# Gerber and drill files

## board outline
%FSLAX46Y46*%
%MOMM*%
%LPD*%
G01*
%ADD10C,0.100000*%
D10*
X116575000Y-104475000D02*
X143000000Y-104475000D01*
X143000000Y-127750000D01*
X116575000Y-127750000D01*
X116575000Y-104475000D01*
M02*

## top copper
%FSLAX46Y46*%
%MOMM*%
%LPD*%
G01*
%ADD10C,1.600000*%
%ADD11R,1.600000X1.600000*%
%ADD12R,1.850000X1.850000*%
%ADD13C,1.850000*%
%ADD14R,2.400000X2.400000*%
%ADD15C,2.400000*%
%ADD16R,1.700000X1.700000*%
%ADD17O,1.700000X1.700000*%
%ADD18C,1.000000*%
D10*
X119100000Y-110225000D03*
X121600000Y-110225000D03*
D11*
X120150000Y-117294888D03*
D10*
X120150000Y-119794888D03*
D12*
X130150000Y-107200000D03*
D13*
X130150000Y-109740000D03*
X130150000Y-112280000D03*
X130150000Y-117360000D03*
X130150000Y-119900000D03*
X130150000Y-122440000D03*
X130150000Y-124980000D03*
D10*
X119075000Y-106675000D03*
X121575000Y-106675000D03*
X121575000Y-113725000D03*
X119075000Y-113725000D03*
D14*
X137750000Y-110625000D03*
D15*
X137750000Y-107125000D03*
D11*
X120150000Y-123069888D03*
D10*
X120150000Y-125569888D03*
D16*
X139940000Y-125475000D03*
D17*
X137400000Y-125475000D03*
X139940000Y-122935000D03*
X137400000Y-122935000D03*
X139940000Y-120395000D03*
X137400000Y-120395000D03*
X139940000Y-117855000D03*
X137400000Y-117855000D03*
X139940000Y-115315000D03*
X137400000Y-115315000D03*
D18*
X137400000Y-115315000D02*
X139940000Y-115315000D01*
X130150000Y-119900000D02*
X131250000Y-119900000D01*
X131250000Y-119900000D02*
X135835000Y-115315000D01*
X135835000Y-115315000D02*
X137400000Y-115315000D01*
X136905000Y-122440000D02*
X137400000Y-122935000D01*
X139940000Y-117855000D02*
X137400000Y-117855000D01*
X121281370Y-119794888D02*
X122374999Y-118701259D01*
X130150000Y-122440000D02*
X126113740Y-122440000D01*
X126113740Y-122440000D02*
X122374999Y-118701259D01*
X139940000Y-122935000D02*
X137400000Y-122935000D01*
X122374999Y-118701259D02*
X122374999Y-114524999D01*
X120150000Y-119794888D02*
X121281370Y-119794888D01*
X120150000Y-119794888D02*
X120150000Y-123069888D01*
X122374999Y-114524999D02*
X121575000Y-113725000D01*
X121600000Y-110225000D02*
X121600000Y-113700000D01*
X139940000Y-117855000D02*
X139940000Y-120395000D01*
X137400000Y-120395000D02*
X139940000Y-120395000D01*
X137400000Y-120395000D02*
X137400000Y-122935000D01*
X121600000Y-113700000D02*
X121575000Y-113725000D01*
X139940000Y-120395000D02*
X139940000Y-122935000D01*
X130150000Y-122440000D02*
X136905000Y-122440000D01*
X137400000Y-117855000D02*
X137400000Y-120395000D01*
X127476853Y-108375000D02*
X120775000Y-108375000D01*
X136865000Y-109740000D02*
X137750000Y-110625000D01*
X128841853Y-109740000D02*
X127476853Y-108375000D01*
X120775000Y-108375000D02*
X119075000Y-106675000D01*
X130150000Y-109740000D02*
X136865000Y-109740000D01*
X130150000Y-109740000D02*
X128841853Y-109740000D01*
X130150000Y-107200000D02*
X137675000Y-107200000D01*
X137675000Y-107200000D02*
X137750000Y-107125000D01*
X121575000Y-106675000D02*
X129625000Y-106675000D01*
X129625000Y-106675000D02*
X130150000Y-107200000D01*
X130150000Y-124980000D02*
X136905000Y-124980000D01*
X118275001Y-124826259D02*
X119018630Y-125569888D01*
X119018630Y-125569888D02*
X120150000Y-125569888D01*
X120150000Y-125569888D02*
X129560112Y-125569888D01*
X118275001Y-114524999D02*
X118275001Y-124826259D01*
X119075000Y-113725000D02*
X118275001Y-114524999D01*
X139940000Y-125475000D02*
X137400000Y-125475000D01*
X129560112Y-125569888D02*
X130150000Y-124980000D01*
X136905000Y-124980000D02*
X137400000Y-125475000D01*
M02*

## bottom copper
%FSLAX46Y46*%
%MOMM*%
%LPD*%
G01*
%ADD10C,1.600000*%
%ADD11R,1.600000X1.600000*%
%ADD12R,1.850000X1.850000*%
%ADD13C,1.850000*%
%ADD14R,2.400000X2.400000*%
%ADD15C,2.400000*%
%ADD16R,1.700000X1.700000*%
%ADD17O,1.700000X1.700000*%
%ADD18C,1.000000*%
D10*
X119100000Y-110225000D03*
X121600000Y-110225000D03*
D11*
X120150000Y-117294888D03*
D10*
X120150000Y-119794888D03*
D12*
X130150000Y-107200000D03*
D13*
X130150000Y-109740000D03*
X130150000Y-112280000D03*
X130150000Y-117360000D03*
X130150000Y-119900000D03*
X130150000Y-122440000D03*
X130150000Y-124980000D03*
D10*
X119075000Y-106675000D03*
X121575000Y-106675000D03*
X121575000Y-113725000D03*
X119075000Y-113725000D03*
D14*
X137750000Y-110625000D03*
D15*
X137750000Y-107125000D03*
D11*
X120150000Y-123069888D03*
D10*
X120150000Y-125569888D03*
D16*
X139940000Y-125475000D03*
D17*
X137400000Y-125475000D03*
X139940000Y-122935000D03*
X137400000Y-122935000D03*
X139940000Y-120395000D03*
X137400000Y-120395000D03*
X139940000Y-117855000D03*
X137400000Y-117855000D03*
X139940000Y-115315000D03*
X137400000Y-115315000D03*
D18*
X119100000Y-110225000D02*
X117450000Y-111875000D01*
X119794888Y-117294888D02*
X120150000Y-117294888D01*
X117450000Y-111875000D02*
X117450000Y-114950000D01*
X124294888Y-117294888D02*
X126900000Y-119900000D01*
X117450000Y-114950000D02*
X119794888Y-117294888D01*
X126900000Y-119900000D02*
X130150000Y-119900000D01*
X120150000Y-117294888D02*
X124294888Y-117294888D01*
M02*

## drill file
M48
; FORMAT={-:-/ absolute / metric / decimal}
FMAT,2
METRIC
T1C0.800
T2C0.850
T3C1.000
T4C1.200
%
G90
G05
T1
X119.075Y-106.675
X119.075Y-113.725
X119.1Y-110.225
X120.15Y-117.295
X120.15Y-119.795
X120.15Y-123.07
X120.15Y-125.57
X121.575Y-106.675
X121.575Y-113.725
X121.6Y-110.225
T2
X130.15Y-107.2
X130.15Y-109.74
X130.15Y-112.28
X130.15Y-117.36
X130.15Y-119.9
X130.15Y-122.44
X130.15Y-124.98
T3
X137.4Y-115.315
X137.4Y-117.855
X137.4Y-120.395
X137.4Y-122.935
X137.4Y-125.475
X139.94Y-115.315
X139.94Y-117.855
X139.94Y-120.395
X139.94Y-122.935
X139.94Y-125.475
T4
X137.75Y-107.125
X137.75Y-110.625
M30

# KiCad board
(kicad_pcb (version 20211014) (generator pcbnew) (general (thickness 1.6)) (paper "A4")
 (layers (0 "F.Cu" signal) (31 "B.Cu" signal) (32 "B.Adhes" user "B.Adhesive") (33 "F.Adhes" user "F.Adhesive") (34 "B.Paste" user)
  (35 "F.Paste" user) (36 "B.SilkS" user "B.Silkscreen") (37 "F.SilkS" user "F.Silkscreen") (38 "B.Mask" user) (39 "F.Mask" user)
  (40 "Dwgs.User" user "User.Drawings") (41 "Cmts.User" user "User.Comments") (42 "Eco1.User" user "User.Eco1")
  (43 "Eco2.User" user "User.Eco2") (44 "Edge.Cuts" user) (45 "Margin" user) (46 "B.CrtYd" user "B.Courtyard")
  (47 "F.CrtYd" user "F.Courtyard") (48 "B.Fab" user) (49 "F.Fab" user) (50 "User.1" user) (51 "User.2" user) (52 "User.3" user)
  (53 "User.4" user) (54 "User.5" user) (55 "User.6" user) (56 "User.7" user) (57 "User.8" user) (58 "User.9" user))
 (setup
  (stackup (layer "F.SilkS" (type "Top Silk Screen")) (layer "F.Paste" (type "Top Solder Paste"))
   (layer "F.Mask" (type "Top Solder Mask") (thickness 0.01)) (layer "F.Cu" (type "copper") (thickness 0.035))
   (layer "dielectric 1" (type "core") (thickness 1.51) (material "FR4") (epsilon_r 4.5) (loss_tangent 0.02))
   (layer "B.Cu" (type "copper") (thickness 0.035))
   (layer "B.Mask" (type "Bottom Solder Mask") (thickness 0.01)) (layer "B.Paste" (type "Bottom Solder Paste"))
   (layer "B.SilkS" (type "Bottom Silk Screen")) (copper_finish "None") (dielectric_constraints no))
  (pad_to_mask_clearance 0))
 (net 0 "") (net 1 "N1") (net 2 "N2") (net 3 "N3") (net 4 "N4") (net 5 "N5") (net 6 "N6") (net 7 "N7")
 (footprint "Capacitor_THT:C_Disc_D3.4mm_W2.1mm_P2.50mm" (layer "F.Cu") (at 119.1 110.225)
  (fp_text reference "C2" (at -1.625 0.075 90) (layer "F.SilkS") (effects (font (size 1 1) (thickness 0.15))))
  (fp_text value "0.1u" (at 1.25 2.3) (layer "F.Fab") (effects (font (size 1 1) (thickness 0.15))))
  (pad "1" thru_hole circle locked (at 0 0) (size 1.6 1.6) (drill 0.8) (layers *.Cu *.Mask) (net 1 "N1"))
  (pad "2" thru_hole circle locked (at 2.5 0) (size 1.6 1.6) (drill 0.8) (layers *.Cu *.Mask) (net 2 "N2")))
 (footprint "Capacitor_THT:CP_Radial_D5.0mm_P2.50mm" (layer "F.Cu") (at 120.15 117.294888 -90)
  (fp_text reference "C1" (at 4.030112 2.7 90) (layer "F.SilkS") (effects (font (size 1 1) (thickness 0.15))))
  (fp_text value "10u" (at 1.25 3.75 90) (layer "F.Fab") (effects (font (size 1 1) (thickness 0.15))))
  (pad "1" thru_hole rect locked (at 0 0 270) (size 1.6 1.6) (drill 0.8) (layers *.Cu *.Mask) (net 1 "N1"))
  (pad "2" thru_hole circle locked (at 2.5 0 270) (size 1.6 1.6) (drill 0.8) (layers *.Cu *.Mask) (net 2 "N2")))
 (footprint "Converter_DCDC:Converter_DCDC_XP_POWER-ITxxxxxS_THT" (layer "F.Cu") (at 130.15 107.2)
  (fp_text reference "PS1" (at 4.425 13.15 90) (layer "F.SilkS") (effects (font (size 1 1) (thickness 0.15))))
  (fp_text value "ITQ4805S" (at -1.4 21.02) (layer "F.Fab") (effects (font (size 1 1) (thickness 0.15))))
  (pad "1" thru_hole rect locked (at 0 0) (size 1.85 1.85) (drill 0.85) (layers *.Cu *.Mask) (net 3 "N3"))
  (pad "2" thru_hole circle locked (at 0 2.54) (size 1.85 1.85) (drill 0.85) (layers *.Cu *.Mask) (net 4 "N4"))
  (pad "3" thru_hole circle locked (at 0 5.08) (size 1.85 1.85) (drill 0.85) (layers *.Cu *.Mask) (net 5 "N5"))
  (pad "5" thru_hole circle locked (at 0 10.16) (size 1.85 1.85) (drill 0.85) (layers *.Cu *.Mask) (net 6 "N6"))
  (pad "6" thru_hole circle locked (at 0 12.7) (size 1.85 1.85) (drill 0.85) (layers *.Cu *.Mask) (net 1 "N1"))
  (pad "7" thru_hole circle locked (at 0 15.24) (size 1.85 1.85) (drill 0.85) (layers *.Cu *.Mask) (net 2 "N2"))
  (pad "8" thru_hole circle locked (at 0 17.78) (size 1.85 1.85) (drill 0.85) (layers *.Cu *.Mask) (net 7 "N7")))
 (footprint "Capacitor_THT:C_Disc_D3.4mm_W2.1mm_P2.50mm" (layer "F.Cu") (at 119.075 106.675)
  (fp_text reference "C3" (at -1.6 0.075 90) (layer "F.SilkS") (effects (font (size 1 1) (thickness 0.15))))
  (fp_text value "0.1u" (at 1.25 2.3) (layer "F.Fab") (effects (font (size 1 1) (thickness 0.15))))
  (pad "1" thru_hole circle locked (at 0 0) (size 1.6 1.6) (drill 0.8) (layers *.Cu *.Mask) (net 4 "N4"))
  (pad "2" thru_hole circle locked (at 2.5 0) (size 1.6 1.6) (drill 0.8) (layers *.Cu *.Mask) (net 3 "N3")))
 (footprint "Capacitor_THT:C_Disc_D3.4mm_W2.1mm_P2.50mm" (layer "F.Cu") (at 121.575 113.725 180)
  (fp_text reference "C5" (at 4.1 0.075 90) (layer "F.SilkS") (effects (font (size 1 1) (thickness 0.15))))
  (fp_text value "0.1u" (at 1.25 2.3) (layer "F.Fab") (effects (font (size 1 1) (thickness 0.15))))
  (pad "1" thru_hole circle locked (at 0 0 180) (size 1.6 1.6) (drill 0.8) (layers *.Cu *.Mask) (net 2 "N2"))
  (pad "2" thru_hole circle locked (at 2.5 0 180) (size 1.6 1.6) (drill 0.8) (layers *.Cu *.Mask) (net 7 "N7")))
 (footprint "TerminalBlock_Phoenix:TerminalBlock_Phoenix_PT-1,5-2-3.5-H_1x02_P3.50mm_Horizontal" (layer "F.Cu") (at 137.75 110.625 90)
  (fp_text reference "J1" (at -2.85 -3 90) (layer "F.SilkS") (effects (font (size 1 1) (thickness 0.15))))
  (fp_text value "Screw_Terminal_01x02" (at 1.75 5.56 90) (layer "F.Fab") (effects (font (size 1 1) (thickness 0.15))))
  (pad "1" thru_hole rect locked (at 0 0 90) (size 2.4 2.4) (drill 1.2) (layers *.Cu *.Mask) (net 4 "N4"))
  (pad "2" thru_hole circle locked (at 3.5 0 90) (size 2.4 2.4) (drill 1.2) (layers *.Cu *.Mask) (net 3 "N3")))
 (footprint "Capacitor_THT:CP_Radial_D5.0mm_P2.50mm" (layer "F.Cu") (at 120.15 123.069888 -90)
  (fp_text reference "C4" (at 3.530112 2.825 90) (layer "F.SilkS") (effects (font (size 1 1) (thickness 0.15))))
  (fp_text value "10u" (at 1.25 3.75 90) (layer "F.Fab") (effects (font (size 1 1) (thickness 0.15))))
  (pad "1" thru_hole rect locked (at 0 0 270) (size 1.6 1.6) (drill 0.8) (layers *.Cu *.Mask) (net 2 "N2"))
  (pad "2" thru_hole circle locked (at 2.5 0 270) (size 1.6 1.6) (drill 0.8) (layers *.Cu *.Mask) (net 7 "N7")))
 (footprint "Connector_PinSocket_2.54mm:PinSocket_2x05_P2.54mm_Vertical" (layer "B.Cu") (at 139.94 125.475)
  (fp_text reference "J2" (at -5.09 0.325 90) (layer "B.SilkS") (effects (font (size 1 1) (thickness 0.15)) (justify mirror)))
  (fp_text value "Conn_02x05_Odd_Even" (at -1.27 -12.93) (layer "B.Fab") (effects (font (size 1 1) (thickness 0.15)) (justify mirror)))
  (pad "1" thru_hole rect locked (at 0 0) (size 1.7 1.7) (drill 1) (layers *.Cu *.Mask) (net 7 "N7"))
  (pad "2" thru_hole oval locked (at -2.54 0) (size 1.7 1.7) (drill 1) (layers *.Cu *.Mask) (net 7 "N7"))
  (pad "3" thru_hole oval locked (at 0 -2.54) (size 1.7 1.7) (drill 1) (layers *.Cu *.Mask) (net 2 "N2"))
  (pad "4" thru_hole oval locked (at -2.54 -2.54) (size 1.7 1.7) (drill 1) (layers *.Cu *.Mask) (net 2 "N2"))
  (pad "5" thru_hole oval locked (at 0 -5.08) (size 1.7 1.7) (drill 1) (layers *.Cu *.Mask) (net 2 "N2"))
  (pad "6" thru_hole oval locked (at -2.54 -5.08) (size 1.7 1.7) (drill 1) (layers *.Cu *.Mask) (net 2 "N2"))
  (pad "7" thru_hole oval locked (at 0 -7.62) (size 1.7 1.7) (drill 1) (layers *.Cu *.Mask) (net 2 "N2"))
  (pad "8" thru_hole oval locked (at -2.54 -7.62) (size 1.7 1.7) (drill 1) (layers *.Cu *.Mask) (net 2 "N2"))
  (pad "9" thru_hole oval locked (at 0 -10.16) (size 1.7 1.7) (drill 1) (layers *.Cu *.Mask) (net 1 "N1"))
  (pad "10" thru_hole oval locked (at -2.54 -10.16) (size 1.7 1.7) (drill 1) (layers *.Cu *.Mask) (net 1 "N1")))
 (gr_rect (start 116.575 104.475) (end 143 127.75) (layer "Edge.Cuts") (width 0.1) (fill none))
 (segment (start 137.4 115.315) (end 139.94 115.315) (width 1) (layer "F.Cu") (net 1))
 (segment (start 130.15 119.9) (end 131.25 119.9) (width 1) (layer "F.Cu") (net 1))
 (segment (start 131.25 119.9) (end 135.835 115.315) (width 1) (layer "F.Cu") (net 1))
 (segment (start 135.835 115.315) (end 137.4 115.315) (width 1) (layer "F.Cu") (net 1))
 (segment (start 119.1 110.225) (end 117.45 111.875) (width 1) (layer "B.Cu") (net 1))
 (segment (start 119.794888 117.294888) (end 120.15 117.294888) (width 1) (layer "B.Cu") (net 1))
 (segment (start 117.45 111.875) (end 117.45 114.95) (width 1) (layer "B.Cu") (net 1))
 (segment (start 124.294888 117.294888) (end 126.9 119.9) (width 1) (layer "B.Cu") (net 1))
 (segment (start 117.45 114.95) (end 119.794888 117.294888) (width 1) (layer "B.Cu") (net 1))
 (segment (start 126.9 119.9) (end 130.15 119.9) (width 1) (layer "B.Cu") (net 1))
 (segment (start 120.15 117.294888) (end 124.294888 117.294888) (width 1) (layer "B.Cu") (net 1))
 (segment (start 136.905 122.44) (end 137.4 122.935) (width 1) (layer "F.Cu") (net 2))
 (segment (start 139.94 117.855) (end 137.4 117.855) (width 1) (layer "F.Cu") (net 2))
 (segment (start 121.28137 119.794888) (end 122.374999 118.701259) (width 1) (layer "F.Cu") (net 2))
 (segment (start 130.15 122.44) (end 126.11374 122.44) (width 1) (layer "F.Cu") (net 2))
 (segment (start 126.11374 122.44) (end 122.374999 118.701259) (width 1) (layer "F.Cu") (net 2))
 (segment (start 139.94 122.935) (end 137.4 122.935) (width 1) (layer "F.Cu") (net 2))
 (segment (start 122.374999 118.701259) (end 122.374999 114.524999) (width 1) (layer "F.Cu") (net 2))
 (segment (start 120.15 119.794888) (end 121.28137 119.794888) (width 1) (layer "F.Cu") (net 2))
 (segment (start 120.15 119.794888) (end 120.15 123.069888) (width 1) (layer "F.Cu") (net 2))
 (segment (start 122.374999 114.524999) (end 121.575 113.725) (width 1) (layer "F.Cu") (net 2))
 (segment (start 121.6 110.225) (end 121.6 113.7) (width 1) (layer "F.Cu") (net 2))
 (segment (start 139.94 117.855) (end 139.94 120.395) (width 1) (layer "F.Cu") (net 2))
 (segment (start 137.4 120.395) (end 139.94 120.395) (width 1) (layer "F.Cu") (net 2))
 (segment (start 137.4 120.395) (end 137.4 122.935) (width 1) (layer "F.Cu") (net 2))
 (segment (start 121.6 113.7) (end 121.575 113.725) (width 1) (layer "F.Cu") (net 2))
 (segment (start 139.94 120.395) (end 139.94 122.935) (width 1) (layer "F.Cu") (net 2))
 (segment (start 130.15 122.44) (end 136.905 122.44) (width 1) (layer "F.Cu") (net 2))
 (segment (start 137.4 117.855) (end 137.4 120.395) (width 1) (layer "F.Cu") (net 2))
 (segment (start 127.476853 108.375) (end 120.775 108.375) (width 1) (layer "F.Cu") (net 4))
 (segment (start 136.865 109.74) (end 137.75 110.625) (width 1) (layer "F.Cu") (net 4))
 (segment (start 128.841853 109.74) (end 127.476853 108.375) (width 1) (layer "F.Cu") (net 4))
 (segment (start 120.775 108.375) (end 119.075 106.675) (width 1) (layer "F.Cu") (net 4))
 (segment (start 130.15 109.74) (end 136.865 109.74) (width 1) (layer "F.Cu") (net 4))
 (segment (start 130.15 109.74) (end 128.841853 109.74) (width 1) (layer "F.Cu") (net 4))
 (segment (start 130.15 107.2) (end 137.675 107.2) (width 1) (layer "F.Cu") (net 3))
 (segment (start 137.675 107.2) (end 137.75 107.125) (width 1) (layer "F.Cu") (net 3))
 (segment (start 121.575 106.675) (end 129.625 106.675) (width 1) (layer "F.Cu") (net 3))
 (segment (start 129.625 106.675) (end 130.15 107.2) (width 1) (layer "F.Cu") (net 3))
 (segment (start 130.15 124.98) (end 136.905 124.98) (width 1) (layer "F.Cu") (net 7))
 (segment (start 118.275001 124.826259) (end 119.01863 125.569888) (width 1) (layer "F.Cu") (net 7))
 (segment (start 119.01863 125.569888) (end 120.15 125.569888) (width 1) (layer "F.Cu") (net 7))
 (segment (start 120.15 125.569888) (end 129.560112 125.569888) (width 1) (layer "F.Cu") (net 7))
 (segment (start 118.275001 114.524999) (end 118.275001 124.826259) (width 1) (layer "F.Cu") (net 7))
 (segment (start 119.075 113.725) (end 118.275001 114.524999) (width 1) (layer "F.Cu") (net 7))
 (segment (start 139.94 125.475) (end 137.4 125.475) (width 1) (layer "F.Cu") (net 7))
 (segment (start 129.560112 125.569888) (end 130.15 124.98) (width 1) (layer "F.Cu") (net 7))
 (segment (start 136.905 124.98) (end 137.4 125.475) (width 1) (layer "F.Cu") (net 7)))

